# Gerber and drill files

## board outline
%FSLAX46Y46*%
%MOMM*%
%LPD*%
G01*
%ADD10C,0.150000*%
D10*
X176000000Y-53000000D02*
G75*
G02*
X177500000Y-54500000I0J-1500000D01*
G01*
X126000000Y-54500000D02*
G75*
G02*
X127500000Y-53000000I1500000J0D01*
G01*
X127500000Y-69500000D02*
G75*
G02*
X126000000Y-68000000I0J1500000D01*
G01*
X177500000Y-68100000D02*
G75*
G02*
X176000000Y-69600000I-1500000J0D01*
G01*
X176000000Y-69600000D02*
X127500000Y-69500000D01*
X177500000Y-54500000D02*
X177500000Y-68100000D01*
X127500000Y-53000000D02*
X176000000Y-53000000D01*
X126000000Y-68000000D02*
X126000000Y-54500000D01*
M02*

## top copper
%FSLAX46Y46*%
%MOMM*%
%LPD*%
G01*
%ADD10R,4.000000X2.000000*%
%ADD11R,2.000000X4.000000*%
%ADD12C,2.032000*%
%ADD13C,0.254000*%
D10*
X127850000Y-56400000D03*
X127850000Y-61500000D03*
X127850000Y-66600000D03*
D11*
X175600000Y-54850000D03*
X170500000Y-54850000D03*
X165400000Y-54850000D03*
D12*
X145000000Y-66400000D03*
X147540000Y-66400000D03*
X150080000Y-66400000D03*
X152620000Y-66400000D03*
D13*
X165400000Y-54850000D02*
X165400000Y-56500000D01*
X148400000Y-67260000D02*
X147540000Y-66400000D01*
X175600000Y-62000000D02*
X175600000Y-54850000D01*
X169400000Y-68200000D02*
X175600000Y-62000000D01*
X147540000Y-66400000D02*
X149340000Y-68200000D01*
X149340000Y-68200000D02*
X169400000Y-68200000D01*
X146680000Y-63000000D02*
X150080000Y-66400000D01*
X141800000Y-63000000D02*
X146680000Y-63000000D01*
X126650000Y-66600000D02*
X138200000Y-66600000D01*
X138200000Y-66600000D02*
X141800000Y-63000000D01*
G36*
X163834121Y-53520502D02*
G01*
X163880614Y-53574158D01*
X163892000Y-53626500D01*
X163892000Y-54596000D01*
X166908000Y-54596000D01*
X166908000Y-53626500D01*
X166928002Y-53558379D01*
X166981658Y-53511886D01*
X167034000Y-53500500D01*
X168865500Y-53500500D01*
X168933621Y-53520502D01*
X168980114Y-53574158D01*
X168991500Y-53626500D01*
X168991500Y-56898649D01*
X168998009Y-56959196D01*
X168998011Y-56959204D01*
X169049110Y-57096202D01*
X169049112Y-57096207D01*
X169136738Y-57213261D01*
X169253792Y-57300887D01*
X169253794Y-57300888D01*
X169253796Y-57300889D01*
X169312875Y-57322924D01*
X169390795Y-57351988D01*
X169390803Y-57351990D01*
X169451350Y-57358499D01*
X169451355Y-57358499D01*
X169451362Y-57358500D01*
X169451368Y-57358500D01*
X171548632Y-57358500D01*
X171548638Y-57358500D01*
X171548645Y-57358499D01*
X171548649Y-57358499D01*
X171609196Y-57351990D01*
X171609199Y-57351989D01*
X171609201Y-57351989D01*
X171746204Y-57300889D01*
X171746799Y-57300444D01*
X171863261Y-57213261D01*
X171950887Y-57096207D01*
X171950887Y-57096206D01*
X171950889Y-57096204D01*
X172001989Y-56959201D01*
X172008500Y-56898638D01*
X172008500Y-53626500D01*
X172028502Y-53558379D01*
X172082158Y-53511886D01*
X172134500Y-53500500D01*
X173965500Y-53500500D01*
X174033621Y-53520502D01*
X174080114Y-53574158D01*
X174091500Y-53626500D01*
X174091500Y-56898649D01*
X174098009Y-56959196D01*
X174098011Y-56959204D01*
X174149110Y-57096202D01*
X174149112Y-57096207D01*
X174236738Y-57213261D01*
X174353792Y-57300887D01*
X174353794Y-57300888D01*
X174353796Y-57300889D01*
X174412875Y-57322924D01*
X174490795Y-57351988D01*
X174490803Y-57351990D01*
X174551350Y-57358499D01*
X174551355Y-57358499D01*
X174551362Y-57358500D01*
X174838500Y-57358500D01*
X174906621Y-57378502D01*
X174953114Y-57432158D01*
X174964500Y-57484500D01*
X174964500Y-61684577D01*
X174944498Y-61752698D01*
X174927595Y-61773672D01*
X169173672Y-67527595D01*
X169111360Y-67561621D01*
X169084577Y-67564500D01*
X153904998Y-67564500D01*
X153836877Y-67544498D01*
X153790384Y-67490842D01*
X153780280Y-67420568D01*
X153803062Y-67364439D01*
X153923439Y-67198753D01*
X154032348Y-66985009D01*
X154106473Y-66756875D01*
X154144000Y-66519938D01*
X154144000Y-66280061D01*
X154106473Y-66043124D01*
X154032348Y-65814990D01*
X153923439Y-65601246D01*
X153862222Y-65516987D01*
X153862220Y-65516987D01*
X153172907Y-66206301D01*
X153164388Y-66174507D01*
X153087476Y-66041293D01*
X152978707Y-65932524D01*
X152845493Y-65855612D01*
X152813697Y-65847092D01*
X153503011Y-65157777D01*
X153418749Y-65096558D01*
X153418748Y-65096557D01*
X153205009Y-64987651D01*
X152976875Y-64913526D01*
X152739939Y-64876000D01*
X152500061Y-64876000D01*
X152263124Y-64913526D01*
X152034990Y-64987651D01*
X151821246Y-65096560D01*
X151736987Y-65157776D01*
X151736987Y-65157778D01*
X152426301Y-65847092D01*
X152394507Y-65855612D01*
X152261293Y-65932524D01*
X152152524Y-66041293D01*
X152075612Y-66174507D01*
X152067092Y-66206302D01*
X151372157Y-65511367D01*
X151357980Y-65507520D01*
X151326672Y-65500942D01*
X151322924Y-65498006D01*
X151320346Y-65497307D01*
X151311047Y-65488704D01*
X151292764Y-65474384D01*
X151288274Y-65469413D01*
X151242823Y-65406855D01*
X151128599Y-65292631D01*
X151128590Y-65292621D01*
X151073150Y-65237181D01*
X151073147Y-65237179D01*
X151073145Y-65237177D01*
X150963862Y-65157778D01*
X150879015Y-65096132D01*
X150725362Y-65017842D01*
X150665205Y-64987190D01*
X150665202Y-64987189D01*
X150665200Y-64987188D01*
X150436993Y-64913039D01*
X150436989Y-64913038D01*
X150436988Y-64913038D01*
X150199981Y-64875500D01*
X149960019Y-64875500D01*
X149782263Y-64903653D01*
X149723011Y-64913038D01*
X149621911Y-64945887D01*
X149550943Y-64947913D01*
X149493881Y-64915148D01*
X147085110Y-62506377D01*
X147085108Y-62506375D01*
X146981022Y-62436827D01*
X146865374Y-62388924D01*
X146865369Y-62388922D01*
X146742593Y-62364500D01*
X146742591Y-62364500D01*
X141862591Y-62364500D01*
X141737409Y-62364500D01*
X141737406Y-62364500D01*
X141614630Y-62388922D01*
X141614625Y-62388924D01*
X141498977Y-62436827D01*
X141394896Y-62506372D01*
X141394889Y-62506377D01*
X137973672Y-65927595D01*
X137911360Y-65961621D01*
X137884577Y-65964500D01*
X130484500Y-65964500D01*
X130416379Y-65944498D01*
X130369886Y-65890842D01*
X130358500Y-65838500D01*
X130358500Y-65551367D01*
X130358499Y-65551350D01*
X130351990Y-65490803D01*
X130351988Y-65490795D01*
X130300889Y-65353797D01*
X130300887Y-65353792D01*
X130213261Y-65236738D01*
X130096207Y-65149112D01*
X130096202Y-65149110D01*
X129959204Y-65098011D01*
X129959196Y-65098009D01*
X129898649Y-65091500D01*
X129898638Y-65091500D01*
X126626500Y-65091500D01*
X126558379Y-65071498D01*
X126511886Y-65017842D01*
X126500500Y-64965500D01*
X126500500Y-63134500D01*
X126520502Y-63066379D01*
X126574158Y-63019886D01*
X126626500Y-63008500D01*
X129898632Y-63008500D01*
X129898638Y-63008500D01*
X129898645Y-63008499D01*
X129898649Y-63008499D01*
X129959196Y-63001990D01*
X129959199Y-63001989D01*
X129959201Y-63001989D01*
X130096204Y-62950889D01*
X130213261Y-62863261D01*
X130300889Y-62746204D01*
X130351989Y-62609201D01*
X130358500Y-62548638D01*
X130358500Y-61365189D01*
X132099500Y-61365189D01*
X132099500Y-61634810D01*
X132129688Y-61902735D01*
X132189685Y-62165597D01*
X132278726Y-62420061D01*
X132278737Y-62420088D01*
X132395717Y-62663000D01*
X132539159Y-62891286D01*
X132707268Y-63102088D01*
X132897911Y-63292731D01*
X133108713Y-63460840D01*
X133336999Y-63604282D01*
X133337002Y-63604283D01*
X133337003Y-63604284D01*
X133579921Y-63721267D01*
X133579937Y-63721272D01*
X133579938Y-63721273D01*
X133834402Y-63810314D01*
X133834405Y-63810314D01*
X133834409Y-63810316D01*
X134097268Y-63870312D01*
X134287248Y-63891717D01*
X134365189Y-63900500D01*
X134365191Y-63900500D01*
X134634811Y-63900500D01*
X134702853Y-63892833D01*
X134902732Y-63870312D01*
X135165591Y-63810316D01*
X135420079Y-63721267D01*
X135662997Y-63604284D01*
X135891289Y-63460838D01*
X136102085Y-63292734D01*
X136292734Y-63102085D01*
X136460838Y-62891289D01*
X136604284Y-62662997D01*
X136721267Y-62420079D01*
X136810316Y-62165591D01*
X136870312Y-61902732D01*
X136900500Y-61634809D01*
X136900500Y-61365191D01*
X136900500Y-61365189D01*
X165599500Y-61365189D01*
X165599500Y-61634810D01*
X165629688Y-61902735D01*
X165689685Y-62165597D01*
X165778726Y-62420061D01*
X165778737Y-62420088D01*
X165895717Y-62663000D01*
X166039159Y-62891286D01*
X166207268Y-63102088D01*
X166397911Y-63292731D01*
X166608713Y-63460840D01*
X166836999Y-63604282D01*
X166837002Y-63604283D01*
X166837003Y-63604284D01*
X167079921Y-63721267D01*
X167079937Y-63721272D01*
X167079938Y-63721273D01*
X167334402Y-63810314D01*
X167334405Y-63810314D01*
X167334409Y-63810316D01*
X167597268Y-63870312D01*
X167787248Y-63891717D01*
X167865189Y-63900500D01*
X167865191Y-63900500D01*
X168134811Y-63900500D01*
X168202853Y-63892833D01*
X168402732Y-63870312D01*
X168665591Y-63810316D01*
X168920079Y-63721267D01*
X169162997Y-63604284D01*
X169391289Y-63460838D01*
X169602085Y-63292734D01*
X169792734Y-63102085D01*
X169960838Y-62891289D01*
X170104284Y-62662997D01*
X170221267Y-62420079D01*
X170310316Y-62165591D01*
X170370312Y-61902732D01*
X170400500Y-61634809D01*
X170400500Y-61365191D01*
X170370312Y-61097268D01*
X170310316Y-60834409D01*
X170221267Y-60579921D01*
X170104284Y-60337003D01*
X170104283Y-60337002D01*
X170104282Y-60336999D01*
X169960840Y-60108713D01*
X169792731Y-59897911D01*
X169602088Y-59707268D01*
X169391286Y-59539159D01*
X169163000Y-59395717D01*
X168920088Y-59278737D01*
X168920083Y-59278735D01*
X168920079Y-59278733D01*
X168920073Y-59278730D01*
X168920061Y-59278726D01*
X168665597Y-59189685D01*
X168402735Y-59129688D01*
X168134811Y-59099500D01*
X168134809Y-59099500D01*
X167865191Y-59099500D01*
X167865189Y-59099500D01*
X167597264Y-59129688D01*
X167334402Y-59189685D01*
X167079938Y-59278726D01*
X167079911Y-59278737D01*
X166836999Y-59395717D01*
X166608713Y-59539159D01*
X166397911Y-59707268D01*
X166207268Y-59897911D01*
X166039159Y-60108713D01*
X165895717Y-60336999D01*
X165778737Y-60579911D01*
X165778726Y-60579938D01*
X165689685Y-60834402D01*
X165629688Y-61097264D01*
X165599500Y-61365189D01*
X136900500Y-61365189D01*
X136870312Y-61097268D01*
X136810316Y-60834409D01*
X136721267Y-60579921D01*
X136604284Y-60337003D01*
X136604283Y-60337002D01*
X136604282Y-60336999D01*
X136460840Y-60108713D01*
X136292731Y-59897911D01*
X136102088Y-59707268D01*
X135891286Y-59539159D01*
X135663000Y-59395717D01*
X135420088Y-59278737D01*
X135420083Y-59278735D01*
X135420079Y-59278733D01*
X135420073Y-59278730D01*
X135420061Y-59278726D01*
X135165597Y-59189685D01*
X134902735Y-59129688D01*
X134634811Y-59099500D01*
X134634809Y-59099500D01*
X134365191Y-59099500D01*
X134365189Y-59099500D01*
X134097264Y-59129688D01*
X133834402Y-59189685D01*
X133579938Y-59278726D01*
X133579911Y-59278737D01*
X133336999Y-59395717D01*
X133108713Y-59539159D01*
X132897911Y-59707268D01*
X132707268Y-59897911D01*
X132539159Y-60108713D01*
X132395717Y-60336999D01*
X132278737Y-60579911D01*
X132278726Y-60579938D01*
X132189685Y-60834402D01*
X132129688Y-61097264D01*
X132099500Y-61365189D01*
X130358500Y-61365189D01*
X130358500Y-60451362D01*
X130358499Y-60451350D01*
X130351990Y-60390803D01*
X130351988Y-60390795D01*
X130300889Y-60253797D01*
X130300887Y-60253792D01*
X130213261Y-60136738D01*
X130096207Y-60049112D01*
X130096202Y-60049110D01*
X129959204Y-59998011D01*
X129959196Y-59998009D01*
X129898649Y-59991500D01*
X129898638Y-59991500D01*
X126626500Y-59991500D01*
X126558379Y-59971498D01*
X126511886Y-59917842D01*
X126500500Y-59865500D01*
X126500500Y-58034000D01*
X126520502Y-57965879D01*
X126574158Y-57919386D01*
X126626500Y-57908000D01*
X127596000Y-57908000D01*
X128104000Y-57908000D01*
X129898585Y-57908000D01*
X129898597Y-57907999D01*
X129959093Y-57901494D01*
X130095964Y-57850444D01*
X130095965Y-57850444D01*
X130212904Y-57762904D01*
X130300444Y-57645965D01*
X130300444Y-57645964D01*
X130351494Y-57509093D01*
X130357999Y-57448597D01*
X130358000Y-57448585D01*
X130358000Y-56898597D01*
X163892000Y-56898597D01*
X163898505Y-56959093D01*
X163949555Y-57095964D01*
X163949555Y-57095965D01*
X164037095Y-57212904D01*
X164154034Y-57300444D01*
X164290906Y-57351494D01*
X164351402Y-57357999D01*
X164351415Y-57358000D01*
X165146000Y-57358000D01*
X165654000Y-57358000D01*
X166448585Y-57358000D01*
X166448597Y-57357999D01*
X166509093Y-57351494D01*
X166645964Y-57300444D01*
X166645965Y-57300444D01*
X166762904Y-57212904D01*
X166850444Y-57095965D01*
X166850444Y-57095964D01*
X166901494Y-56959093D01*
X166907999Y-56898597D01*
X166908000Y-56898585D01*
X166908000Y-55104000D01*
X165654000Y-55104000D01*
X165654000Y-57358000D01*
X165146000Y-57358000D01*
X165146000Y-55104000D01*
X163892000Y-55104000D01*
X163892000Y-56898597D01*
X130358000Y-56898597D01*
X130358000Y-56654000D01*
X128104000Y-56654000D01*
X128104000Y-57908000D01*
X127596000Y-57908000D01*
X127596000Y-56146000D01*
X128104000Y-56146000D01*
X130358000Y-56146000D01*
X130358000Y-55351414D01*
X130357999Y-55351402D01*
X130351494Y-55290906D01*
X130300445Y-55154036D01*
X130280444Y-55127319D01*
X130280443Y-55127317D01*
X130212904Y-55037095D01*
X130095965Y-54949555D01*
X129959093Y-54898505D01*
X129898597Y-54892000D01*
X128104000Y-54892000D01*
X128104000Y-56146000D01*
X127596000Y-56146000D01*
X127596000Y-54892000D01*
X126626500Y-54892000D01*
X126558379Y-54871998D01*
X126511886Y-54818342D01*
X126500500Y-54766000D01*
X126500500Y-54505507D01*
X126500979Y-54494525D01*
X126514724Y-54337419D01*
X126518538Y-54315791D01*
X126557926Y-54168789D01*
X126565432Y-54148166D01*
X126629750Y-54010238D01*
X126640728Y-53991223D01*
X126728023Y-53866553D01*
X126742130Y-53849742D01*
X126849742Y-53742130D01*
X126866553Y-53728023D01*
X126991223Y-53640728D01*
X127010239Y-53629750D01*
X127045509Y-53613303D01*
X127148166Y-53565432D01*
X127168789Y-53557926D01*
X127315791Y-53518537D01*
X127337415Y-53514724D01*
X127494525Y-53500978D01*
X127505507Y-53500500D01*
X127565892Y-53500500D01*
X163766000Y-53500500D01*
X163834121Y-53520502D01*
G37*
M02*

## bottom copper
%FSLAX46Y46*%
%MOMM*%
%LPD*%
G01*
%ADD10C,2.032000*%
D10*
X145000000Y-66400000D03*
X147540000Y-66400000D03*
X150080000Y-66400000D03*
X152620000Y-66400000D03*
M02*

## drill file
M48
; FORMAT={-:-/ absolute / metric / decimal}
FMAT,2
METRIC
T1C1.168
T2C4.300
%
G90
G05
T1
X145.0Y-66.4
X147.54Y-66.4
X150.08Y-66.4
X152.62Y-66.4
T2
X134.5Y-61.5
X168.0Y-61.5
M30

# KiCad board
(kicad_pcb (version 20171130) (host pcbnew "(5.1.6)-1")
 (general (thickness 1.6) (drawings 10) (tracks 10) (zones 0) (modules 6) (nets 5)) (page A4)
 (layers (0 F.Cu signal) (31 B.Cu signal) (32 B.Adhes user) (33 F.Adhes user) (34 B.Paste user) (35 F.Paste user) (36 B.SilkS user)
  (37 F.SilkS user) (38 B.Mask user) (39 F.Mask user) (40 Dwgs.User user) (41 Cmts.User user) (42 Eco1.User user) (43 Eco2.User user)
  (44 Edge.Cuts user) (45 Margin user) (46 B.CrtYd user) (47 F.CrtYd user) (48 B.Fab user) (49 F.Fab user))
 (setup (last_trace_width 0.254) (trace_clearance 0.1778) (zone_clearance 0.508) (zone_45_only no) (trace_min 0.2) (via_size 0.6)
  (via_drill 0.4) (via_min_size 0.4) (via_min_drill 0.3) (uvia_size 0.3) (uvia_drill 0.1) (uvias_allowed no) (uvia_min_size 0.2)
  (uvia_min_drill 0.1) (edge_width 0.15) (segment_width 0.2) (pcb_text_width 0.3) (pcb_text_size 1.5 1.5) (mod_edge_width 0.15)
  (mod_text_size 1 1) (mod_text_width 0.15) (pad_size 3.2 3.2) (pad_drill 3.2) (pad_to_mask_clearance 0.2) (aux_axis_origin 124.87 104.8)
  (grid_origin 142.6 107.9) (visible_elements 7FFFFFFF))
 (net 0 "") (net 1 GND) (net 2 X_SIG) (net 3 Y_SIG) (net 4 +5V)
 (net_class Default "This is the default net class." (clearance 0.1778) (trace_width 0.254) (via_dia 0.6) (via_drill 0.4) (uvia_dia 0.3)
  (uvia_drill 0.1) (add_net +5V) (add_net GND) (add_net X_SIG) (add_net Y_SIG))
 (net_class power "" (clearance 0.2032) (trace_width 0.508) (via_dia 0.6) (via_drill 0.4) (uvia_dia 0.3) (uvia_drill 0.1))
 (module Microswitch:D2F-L (layer F.Cu) (at 119.25 67.9 90)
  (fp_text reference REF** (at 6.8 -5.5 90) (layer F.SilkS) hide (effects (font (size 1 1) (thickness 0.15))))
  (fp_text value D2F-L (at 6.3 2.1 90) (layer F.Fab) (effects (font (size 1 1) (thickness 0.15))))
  (pad 3 connect rect (at 11.5 8.6 90) (size 2 4) (layers F.Cu F.Mask) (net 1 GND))
  (pad 2 connect rect (at 6.4 8.6 90) (size 2 4) (layers F.Cu F.Mask))
  (pad 1 connect rect (at 1.3 8.6 90) (size 2 4) (layers F.Cu F.Mask) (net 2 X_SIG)))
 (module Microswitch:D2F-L (layer F.Cu) (at 164.1 46.25)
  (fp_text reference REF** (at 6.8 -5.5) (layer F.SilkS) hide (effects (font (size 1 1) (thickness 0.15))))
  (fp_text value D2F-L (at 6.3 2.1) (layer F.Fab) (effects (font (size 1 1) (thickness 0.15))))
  (pad 3 connect rect (at 11.5 8.6) (size 2 4) (layers F.Cu F.Mask) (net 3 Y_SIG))
  (pad 2 connect rect (at 6.4 8.6) (size 2 4) (layers F.Cu F.Mask))
  (pad 1 connect rect (at 1.3 8.6) (size 2 4) (layers F.Cu F.Mask) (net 1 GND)))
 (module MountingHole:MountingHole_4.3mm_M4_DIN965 (layer F.Cu) (at 168 61.5)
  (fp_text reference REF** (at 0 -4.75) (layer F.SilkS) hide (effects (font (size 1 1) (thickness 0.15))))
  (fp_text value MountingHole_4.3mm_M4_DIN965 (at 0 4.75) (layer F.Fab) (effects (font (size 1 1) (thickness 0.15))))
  (pad 1 np_thru_hole circle (at 0 0) (size 4.3 4.3) (drill 4.3) (layers *.Cu *.Mask)))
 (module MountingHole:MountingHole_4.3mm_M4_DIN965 (layer F.Cu) (at 134.5 61.5)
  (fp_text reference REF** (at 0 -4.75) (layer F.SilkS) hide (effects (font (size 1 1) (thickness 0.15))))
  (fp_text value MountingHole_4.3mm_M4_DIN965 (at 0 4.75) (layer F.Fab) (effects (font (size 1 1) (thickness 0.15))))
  (pad 1 np_thru_hole circle (at 0 0) (size 4.3 4.3) (drill 4.3) (layers *.Cu *.Mask)))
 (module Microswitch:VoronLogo (layer F.Cu) (at 152.25 61.5)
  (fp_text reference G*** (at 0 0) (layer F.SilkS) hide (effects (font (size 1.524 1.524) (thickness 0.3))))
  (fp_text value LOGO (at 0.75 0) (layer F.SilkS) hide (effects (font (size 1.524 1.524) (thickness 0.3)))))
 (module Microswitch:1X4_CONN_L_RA (layer B.Cu) (at 148.81 66.4 90)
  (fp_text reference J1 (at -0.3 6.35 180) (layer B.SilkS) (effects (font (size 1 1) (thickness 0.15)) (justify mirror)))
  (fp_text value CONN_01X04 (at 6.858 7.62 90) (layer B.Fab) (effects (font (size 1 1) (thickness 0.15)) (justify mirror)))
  (pad 4 thru_hole circle (at 0 -3.81 90) (size 2.032 2.032) (drill 1.1684) (layers *.Cu *.Mask B.SilkS) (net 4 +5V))
  (pad 3 thru_hole circle (at 0 -1.27 90) (size 2.032 2.032) (drill 1.1684) (layers *.Cu *.Mask B.SilkS) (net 3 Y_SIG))
  (pad 2 thru_hole circle (at 0 1.27 90) (size 2.032 2.032) (drill 1.1684) (layers *.Cu *.Mask B.SilkS) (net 2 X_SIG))
  (pad 1 thru_hole circle (at 0 3.81 90) (size 2.032 2.032) (drill 1.1684) (layers *.Cu *.Mask B.SilkS) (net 1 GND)))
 (gr_arc (start 176 54.5) (end 177.5 54.5) (angle -90) (layer Edge.Cuts) (width 0.15))
 (gr_arc (start 127.5 54.5) (end 127.5 53) (angle -90) (layer Edge.Cuts) (width 0.15))
 (gr_arc (start 127.5 68) (end 126 68) (angle -90) (layer Edge.Cuts) (width 0.15))
 (gr_arc (start 176 68.1) (end 176 69.6) (angle -90) (layer Edge.Cuts) (width 0.15))
 (gr_line (start 176 69.6) (end 127.5 69.5) (layer Edge.Cuts) (width 0.15))
 (gr_line (start 177.5 54.5) (end 177.5 68.1) (layer Edge.Cuts) (width 0.15))
 (gr_line (start 127.5 53) (end 176 53) (layer Edge.Cuts) (width 0.15))
 (gr_line (start 126 68) (end 126 54.5) (layer Edge.Cuts) (width 0.15))
 (segment (start 165.4 54.85) (end 165.4 56.5) (width 0.254) (layer F.Cu) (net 1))
 (segment (start 148.4 67.26) (end 147.54 66.4) (width 0.254) (layer F.Cu) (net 3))
 (segment (start 175.6 62) (end 175.6 54.85) (width 0.254) (layer F.Cu) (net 3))
 (segment (start 169.4 68.2) (end 175.6 62) (width 0.254) (layer F.Cu) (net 3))
 (segment (start 147.54 66.4) (end 149.34 68.2) (width 0.254) (layer F.Cu) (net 3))
 (segment (start 149.34 68.2) (end 169.4 68.2) (width 0.254) (layer F.Cu) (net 3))
 (segment (start 146.68 63) (end 150.08 66.4) (width 0.254) (layer F.Cu) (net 2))
 (segment (start 141.8 63) (end 146.68 63) (width 0.254) (layer F.Cu) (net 2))
 (segment (start 126.65 66.6) (end 138.2 66.6) (width 0.254) (layer F.Cu) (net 2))
 (segment (start 138.2 66.6) (end 141.8 63) (width 0.254) (layer F.Cu) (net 2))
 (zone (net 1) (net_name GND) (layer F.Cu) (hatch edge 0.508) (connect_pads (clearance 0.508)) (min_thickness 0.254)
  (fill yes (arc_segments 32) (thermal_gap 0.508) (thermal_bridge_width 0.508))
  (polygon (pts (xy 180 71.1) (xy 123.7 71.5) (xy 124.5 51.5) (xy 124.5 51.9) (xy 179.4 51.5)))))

